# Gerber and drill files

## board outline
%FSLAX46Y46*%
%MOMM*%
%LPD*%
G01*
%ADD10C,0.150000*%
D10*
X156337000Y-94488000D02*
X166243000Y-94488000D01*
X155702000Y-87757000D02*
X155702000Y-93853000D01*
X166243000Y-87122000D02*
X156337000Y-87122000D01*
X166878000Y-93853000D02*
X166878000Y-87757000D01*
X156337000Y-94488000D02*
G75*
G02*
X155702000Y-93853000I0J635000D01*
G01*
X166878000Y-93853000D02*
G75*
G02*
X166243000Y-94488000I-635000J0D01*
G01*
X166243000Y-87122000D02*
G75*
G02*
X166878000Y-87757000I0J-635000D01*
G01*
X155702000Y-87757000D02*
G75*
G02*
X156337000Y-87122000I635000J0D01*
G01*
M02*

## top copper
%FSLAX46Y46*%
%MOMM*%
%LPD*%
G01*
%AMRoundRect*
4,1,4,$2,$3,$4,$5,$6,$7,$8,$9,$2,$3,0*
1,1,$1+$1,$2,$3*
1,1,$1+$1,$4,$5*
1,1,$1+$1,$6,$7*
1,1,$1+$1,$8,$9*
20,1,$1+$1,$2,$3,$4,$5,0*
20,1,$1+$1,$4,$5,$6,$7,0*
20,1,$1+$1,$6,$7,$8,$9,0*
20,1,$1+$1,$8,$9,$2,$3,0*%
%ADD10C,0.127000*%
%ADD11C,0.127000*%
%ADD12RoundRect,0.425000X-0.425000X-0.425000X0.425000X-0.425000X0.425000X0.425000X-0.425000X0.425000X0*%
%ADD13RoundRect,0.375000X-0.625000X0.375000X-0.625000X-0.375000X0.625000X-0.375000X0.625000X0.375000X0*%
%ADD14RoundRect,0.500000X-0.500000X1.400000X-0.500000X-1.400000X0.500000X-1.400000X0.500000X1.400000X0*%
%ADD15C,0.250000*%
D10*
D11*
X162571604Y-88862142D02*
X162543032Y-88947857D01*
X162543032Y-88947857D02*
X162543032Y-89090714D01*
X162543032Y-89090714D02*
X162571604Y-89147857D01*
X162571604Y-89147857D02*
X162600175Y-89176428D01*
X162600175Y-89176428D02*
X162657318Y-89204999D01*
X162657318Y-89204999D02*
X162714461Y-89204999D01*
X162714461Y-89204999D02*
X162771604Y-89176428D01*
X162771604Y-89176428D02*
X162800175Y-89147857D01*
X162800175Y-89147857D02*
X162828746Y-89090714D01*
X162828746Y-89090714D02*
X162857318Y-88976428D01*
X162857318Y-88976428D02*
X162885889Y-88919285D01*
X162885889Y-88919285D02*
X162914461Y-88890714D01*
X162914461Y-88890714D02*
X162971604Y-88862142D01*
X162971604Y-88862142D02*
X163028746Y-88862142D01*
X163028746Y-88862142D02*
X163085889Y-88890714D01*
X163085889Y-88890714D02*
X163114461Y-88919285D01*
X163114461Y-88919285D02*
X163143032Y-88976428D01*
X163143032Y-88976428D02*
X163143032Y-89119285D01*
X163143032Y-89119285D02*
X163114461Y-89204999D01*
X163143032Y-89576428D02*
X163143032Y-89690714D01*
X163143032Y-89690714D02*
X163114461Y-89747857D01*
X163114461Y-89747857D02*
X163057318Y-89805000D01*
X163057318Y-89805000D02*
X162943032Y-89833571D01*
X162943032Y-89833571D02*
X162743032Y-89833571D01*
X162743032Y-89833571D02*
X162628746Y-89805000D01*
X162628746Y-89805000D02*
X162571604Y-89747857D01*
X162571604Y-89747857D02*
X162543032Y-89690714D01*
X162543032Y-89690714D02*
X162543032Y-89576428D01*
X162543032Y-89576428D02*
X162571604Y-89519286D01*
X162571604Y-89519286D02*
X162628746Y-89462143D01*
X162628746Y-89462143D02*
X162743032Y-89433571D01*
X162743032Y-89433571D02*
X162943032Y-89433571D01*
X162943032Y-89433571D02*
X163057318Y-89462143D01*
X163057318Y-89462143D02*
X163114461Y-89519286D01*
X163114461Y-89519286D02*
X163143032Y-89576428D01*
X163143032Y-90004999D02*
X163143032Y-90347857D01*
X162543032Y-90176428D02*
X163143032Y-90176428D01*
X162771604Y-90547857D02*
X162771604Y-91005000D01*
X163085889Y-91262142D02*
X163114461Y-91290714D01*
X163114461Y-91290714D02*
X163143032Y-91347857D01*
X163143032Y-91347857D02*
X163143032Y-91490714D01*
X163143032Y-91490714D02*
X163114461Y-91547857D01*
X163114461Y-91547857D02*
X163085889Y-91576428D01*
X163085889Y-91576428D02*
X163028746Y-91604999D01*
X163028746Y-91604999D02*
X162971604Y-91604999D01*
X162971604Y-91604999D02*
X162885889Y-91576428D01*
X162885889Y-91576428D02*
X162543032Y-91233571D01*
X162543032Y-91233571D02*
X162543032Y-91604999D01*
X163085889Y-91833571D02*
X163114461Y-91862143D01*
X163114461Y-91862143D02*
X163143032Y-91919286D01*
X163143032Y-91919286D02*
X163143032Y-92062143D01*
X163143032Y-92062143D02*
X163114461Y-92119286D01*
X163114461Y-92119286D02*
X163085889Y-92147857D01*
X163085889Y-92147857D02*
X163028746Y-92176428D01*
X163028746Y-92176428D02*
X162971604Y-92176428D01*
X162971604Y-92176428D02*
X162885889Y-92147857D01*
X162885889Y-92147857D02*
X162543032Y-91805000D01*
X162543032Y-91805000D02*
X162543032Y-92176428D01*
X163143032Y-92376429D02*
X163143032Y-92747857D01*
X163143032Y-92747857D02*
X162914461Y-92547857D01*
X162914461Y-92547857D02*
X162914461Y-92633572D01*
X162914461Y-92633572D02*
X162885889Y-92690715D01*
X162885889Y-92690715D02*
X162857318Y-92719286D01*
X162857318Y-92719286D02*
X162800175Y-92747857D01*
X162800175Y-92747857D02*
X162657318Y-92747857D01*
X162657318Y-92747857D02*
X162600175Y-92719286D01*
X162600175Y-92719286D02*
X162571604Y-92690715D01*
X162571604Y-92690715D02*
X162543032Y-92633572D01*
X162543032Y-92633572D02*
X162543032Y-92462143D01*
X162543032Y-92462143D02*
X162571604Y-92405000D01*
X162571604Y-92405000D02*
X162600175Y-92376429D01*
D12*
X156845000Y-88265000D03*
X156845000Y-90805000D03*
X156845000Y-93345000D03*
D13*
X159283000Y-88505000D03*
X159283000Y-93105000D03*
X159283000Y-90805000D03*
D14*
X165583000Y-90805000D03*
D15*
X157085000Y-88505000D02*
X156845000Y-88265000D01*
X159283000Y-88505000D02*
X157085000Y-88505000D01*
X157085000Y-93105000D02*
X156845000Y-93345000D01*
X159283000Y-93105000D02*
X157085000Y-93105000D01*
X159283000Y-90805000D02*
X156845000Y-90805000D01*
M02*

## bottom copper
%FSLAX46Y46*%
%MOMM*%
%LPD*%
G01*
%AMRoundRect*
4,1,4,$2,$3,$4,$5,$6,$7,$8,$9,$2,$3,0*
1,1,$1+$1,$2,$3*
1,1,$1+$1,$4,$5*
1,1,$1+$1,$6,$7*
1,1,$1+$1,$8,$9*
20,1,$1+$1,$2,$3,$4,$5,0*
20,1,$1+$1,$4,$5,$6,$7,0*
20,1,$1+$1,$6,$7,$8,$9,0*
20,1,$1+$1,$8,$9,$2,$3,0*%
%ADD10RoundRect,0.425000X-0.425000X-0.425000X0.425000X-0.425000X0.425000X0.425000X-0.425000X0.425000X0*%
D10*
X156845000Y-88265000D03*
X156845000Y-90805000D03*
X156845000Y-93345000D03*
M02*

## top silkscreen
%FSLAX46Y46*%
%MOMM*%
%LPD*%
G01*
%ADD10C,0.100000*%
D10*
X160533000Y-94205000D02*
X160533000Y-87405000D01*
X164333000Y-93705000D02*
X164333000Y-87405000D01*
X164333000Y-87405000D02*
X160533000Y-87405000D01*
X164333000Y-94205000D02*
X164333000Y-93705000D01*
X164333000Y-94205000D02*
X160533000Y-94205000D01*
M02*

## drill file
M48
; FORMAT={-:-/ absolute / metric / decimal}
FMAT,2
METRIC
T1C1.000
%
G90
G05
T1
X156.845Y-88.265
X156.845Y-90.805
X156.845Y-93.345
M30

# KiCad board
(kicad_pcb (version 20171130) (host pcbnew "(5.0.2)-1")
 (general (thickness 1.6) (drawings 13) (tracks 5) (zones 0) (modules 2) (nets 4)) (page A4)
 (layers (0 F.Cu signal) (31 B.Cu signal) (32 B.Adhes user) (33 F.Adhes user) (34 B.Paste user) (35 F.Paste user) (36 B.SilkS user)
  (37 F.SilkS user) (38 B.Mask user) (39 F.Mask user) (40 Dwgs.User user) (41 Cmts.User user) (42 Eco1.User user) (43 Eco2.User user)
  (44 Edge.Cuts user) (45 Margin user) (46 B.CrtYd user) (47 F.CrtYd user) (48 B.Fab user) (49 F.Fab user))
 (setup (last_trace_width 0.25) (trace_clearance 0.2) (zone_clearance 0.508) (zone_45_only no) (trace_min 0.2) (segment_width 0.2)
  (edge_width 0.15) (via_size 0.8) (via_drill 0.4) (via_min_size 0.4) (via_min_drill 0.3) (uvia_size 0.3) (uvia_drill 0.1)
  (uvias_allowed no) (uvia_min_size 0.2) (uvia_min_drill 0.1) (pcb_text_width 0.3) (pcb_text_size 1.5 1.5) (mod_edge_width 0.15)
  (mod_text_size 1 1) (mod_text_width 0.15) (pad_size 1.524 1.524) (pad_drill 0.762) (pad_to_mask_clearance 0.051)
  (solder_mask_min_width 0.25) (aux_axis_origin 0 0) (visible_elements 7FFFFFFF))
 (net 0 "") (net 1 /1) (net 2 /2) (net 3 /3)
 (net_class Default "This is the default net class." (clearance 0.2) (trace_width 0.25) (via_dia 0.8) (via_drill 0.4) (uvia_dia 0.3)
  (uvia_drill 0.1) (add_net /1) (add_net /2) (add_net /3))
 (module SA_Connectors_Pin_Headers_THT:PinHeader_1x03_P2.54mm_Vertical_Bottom (layer F.Cu) (at 156.845 88.265)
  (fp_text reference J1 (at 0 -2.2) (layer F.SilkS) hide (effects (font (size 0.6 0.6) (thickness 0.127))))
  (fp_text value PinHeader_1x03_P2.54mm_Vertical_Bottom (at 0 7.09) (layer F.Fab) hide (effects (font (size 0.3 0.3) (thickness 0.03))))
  (pad 1 thru_hole roundrect (at 0 0) (size 1.7 1.7) (drill 1) (layers *.Cu *.Mask) (roundrect_rratio 0.25) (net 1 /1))
  (pad 2 thru_hole roundrect (at 0 2.54) (size 1.7 1.7) (drill 1) (layers *.Cu *.Mask) (roundrect_rratio 0.25) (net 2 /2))
  (pad 3 thru_hole roundrect (at 0 5.08) (size 1.7 1.7) (drill 1) (layers *.Cu *.Mask) (roundrect_rratio 0.25) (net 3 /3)))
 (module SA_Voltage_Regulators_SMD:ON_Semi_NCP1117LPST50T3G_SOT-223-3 (layer F.Cu) (at 162.433 90.805 270)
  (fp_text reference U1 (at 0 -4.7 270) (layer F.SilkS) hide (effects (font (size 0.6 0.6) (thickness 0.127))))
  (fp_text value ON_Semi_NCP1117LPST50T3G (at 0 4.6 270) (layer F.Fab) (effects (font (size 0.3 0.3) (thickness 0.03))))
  (fp_line (start 3.4 1.9) (end -3.4 1.9) (layer F.SilkS) (width 0.1))
  (fp_line (start 2.9 -1.9) (end -3.4 -1.9) (layer F.SilkS) (width 0.1))
  (fp_line (start -3.4 -1.9) (end -3.4 1.9) (layer F.SilkS) (width 0.1))
  (fp_line (start 3.4 -1.9) (end 2.9 -1.9) (layer F.SilkS) (width 0.1))
  (fp_line (start 3.4 -1.9) (end 3.4 1.9) (layer F.SilkS) (width 0.1))
  (pad 1 smd roundrect (at -2.3 3.15 270) (size 1.5 2) (layers F.Cu F.Paste F.Mask) (roundrect_rratio 0.25) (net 1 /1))
  (pad 3 smd roundrect (at 2.3 3.15 270) (size 1.5 2) (layers F.Cu F.Paste F.Mask) (roundrect_rratio 0.25) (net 3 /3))
  (pad 2 smd roundrect (at 0 3.15 270) (size 1.5 2) (layers F.Cu F.Paste F.Mask) (roundrect_rratio 0.25) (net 2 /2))
  (pad 2 smd roundrect (at 0 -3.15 270) (size 3.8 2) (layers F.Cu F.Paste F.Mask) (roundrect_rratio 0.25) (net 2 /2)))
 (gr_line (start 156.337 94.488) (end 166.243 94.488) (layer Edge.Cuts) (width 0.15))
 (gr_line (start 155.702 87.757) (end 155.702 93.853) (layer Edge.Cuts) (width 0.15))
 (gr_line (start 166.243 87.122) (end 156.337 87.122) (layer Edge.Cuts) (width 0.15))
 (gr_line (start 166.878 93.853) (end 166.878 87.757) (layer Edge.Cuts) (width 0.15))
 (gr_arc (start 156.337 93.853) (end 155.702 93.853) (angle -90) (layer Edge.Cuts) (width 0.15))
 (gr_arc (start 166.243 93.853) (end 166.243 94.488) (angle -90) (layer Edge.Cuts) (width 0.15))
 (gr_arc (start 166.243 87.757) (end 166.878 87.757) (angle -90) (layer Edge.Cuts) (width 0.15))
 (gr_arc (start 156.337 87.757) (end 156.337 87.122) (angle -90) (layer Edge.Cuts) (width 0.15))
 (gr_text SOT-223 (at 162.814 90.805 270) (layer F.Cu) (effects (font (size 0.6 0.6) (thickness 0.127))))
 (segment (start 157.085 88.505) (end 156.845 88.265) (width 0.25) (layer F.Cu) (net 1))
 (segment (start 159.283 88.505) (end 157.085 88.505) (width 0.25) (layer F.Cu) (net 1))
 (segment (start 157.085 93.105) (end 156.845 93.345) (width 0.25) (layer F.Cu) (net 3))
 (segment (start 159.283 93.105) (end 157.085 93.105) (width 0.25) (layer F.Cu) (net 3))
 (segment (start 159.283 90.805) (end 156.845 90.805) (width 0.25) (layer F.Cu) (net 2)))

